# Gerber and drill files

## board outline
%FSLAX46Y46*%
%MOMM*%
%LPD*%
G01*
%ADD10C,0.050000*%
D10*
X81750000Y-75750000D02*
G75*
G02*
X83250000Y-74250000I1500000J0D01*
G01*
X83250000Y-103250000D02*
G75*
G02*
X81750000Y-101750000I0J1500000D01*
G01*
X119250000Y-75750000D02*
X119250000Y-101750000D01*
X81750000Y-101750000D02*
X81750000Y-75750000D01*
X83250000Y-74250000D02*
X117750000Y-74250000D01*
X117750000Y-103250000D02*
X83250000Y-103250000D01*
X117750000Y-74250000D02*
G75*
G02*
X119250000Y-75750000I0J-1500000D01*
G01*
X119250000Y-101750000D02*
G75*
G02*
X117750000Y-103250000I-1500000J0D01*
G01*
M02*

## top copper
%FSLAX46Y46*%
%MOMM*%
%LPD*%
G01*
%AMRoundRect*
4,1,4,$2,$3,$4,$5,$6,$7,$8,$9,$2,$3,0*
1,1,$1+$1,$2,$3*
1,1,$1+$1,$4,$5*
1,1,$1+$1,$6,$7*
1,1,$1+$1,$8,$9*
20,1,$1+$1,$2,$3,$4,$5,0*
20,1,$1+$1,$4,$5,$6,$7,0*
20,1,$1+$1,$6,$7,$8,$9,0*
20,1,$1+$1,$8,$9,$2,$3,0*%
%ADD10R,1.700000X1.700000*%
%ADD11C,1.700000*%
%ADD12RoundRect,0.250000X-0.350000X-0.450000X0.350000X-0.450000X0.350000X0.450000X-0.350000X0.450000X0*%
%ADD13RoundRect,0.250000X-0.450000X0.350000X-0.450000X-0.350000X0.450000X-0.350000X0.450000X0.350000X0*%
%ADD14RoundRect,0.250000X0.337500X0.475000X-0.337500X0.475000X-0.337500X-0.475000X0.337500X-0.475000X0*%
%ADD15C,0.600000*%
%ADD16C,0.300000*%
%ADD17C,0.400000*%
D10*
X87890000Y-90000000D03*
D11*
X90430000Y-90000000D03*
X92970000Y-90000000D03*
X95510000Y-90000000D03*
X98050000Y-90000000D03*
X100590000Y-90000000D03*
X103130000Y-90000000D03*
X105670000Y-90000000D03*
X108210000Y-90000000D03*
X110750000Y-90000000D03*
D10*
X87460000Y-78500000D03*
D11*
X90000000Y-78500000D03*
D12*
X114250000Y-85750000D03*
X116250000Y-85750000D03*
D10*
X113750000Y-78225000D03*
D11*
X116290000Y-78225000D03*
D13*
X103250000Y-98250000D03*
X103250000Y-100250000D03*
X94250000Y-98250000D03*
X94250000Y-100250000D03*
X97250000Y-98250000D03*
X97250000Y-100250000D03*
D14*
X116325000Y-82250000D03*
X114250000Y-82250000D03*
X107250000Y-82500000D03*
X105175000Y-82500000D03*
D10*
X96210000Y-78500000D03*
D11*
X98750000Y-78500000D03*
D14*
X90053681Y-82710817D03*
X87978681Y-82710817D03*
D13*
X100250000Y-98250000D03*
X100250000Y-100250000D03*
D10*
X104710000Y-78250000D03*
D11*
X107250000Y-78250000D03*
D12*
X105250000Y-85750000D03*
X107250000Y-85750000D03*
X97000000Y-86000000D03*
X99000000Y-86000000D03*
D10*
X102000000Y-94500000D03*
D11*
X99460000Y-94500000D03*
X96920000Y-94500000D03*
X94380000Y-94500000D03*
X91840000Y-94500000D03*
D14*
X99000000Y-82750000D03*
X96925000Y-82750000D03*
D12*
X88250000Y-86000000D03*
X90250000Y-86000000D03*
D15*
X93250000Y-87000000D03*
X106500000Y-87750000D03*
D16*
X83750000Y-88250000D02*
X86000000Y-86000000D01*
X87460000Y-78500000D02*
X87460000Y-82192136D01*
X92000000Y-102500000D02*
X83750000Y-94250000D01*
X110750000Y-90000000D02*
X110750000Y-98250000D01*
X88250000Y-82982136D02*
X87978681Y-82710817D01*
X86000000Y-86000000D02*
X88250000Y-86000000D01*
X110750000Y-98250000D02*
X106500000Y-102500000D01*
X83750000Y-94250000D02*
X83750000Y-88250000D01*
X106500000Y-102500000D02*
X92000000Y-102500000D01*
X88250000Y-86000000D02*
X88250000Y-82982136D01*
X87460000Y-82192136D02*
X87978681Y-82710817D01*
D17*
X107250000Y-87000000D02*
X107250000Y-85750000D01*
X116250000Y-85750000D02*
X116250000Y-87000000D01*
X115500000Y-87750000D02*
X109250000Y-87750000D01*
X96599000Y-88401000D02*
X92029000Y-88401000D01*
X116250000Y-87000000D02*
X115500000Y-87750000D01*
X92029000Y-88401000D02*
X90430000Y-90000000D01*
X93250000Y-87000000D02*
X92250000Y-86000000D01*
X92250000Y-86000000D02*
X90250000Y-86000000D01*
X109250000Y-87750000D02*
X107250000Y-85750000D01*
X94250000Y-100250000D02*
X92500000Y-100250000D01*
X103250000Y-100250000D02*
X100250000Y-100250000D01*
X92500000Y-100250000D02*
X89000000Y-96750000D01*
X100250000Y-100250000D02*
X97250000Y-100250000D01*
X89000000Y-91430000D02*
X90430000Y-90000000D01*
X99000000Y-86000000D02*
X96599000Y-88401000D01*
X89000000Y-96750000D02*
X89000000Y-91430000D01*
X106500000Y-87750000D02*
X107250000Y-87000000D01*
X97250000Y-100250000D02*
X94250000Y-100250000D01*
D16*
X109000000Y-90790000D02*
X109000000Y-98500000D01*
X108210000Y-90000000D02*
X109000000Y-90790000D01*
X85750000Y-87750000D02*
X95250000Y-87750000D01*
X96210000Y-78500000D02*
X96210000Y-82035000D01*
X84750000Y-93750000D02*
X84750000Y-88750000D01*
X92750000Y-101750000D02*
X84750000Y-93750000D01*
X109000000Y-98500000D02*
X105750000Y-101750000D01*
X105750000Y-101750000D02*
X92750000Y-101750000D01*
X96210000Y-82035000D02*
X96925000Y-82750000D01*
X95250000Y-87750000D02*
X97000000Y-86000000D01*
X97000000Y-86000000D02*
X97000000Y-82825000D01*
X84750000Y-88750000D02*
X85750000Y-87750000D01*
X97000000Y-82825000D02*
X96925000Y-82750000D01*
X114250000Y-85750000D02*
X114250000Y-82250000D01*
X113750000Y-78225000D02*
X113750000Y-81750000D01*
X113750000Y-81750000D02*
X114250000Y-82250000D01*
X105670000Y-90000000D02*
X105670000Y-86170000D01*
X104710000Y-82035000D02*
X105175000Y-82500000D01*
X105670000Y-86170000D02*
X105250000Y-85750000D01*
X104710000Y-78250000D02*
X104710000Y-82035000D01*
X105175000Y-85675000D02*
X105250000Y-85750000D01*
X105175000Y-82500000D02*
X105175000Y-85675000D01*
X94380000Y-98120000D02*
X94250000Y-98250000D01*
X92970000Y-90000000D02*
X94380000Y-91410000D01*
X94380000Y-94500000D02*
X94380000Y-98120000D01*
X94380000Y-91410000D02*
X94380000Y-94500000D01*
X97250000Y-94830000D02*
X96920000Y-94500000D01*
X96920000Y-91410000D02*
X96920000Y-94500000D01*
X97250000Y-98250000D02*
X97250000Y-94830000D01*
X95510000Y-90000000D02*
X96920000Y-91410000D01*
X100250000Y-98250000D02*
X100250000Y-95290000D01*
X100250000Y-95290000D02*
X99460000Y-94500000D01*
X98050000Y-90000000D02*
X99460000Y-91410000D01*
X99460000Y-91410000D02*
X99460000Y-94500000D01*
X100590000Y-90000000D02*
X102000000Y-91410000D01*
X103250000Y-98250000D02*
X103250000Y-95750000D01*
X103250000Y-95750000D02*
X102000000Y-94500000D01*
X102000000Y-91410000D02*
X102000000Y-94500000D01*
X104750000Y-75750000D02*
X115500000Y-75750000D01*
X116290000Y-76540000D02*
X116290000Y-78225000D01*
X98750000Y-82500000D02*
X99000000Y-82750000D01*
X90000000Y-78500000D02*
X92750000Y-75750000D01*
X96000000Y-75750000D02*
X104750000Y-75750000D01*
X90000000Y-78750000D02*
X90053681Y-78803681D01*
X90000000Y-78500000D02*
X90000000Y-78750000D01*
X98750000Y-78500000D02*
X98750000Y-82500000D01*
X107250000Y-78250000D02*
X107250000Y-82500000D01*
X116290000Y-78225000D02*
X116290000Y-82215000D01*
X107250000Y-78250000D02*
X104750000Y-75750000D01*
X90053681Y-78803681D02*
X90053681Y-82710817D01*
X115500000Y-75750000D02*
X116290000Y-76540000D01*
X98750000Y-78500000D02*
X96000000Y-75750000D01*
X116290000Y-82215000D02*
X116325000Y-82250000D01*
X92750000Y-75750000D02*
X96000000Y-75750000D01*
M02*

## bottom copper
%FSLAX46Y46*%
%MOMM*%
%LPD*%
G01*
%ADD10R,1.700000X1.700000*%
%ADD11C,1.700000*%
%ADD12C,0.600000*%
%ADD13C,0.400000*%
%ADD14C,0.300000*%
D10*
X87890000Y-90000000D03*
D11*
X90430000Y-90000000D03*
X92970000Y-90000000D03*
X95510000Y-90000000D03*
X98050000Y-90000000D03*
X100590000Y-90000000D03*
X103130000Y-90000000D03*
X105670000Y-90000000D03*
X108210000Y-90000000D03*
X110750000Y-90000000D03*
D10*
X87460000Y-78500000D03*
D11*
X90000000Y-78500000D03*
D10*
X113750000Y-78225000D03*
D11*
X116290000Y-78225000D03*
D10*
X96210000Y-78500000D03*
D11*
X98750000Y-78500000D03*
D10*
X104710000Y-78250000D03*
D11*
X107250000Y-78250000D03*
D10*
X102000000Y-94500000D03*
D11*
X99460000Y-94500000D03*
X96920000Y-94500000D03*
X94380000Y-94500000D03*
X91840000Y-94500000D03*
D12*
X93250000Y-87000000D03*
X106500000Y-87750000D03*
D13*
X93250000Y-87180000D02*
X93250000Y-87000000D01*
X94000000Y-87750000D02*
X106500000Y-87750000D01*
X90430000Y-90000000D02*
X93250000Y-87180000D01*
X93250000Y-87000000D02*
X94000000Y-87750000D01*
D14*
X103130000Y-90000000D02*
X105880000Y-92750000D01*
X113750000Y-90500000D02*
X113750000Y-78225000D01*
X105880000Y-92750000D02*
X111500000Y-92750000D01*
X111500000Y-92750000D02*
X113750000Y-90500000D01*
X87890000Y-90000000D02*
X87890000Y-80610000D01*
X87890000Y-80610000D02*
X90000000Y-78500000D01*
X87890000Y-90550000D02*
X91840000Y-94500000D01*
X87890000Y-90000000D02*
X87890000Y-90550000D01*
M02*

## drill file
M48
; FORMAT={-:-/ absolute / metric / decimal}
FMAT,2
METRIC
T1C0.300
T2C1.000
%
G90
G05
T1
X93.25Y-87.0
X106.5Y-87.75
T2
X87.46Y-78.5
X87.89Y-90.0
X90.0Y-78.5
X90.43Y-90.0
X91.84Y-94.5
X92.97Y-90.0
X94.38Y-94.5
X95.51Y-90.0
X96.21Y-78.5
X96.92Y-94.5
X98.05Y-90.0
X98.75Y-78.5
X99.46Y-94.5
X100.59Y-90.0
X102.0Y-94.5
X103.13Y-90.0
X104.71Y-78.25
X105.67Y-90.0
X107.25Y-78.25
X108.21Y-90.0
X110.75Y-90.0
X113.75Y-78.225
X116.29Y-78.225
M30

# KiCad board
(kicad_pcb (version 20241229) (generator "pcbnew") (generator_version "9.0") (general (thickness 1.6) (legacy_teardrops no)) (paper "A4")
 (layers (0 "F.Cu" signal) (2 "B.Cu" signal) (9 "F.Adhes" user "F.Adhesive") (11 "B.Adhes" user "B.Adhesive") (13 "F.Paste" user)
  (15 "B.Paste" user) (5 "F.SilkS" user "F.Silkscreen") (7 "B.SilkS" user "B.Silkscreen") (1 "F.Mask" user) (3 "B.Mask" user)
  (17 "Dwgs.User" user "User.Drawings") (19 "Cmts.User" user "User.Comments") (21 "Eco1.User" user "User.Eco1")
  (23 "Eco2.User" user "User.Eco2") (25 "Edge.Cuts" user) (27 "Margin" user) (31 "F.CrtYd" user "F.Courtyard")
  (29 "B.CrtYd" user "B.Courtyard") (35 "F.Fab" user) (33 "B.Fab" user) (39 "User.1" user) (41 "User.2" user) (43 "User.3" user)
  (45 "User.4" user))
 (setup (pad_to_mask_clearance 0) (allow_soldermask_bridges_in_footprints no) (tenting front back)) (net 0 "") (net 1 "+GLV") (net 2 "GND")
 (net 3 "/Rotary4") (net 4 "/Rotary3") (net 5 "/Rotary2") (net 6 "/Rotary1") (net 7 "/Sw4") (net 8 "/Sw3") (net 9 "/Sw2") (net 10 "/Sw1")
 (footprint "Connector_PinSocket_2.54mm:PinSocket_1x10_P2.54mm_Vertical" (layer "F.Cu") (at 87.89 90 90)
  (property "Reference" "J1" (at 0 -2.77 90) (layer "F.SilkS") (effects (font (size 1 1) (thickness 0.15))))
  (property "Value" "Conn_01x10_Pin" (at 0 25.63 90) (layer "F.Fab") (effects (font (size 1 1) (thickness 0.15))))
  (pad "1" thru_hole rect (at 0 0 90) (size 1.7 1.7) (drill 1) (layers "*.Cu" "*.Mask") (remove_unused_layers no) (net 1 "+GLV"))
  (pad "2" thru_hole circle (at 0 2.54 90) (size 1.7 1.7) (drill 1) (layers "*.Cu" "*.Mask") (remove_unused_layers no) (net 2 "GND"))
  (pad "3" thru_hole circle (at 0 5.08 90) (size 1.7 1.7) (drill 1) (layers "*.Cu" "*.Mask") (remove_unused_layers no) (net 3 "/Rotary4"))
  (pad "4" thru_hole circle (at 0 7.62 90) (size 1.7 1.7) (drill 1) (layers "*.Cu" "*.Mask") (remove_unused_layers no) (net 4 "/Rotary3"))
  (pad "5" thru_hole circle (at 0 10.16 90) (size 1.7 1.7) (drill 1) (layers "*.Cu" "*.Mask") (remove_unused_layers no) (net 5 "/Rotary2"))
  (pad "6" thru_hole circle (at 0 12.7 90) (size 1.7 1.7) (drill 1) (layers "*.Cu" "*.Mask") (remove_unused_layers no) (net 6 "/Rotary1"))
  (pad "7" thru_hole circle (at 0 15.24 90) (size 1.7 1.7) (drill 1) (layers "*.Cu" "*.Mask") (remove_unused_layers no) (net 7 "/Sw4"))
  (pad "8" thru_hole circle (at 0 17.78 90) (size 1.7 1.7) (drill 1) (layers "*.Cu" "*.Mask") (remove_unused_layers no) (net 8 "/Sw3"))
  (pad "9" thru_hole circle (at 0 20.32 90) (size 1.7 1.7) (drill 1) (layers "*.Cu" "*.Mask") (remove_unused_layers no) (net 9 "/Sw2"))
  (pad "10" thru_hole circle (at 0 22.86 90) (size 1.7 1.7) (drill 1) (layers "*.Cu" "*.Mask") (remove_unused_layers no) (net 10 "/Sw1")))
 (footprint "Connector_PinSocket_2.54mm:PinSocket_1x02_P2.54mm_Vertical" (layer "F.Cu") (at 87.46 78.5 90)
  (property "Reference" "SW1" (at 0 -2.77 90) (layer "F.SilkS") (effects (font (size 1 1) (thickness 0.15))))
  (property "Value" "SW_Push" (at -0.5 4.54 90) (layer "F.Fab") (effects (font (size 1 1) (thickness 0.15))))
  (pad "1" thru_hole rect (at 0 0 90) (size 1.7 1.7) (drill 1) (layers "*.Cu" "*.Mask") (remove_unused_layers no) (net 10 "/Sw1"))
  (pad "2" thru_hole circle (at 0 2.54 90) (size 1.7 1.7) (drill 1) (layers "*.Cu" "*.Mask") (remove_unused_layers no) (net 1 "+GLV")))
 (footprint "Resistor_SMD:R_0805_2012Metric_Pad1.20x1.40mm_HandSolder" (layer "F.Cu") (at 115.25 85.75)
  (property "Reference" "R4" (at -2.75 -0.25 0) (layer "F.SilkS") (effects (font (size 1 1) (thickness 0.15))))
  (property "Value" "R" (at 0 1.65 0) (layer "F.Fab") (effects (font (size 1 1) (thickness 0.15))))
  (pad "1" smd roundrect (at -1 0) (size 1.2 1.4) (layers "F.Cu" "F.Mask" "F.Paste") (roundrect_rratio 0.208333) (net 7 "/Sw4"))
  (pad "2" smd roundrect (at 1 0) (size 1.2 1.4) (layers "F.Cu" "F.Mask" "F.Paste") (roundrect_rratio 0.208333) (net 2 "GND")))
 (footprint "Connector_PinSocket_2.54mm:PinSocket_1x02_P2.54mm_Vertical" (layer "F.Cu") (at 113.75 78.225 90)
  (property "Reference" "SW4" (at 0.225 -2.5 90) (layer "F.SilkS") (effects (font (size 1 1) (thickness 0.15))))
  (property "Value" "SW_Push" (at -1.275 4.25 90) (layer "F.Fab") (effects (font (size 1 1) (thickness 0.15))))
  (pad "1" thru_hole rect (at 0 0 90) (size 1.7 1.7) (drill 1) (layers "*.Cu" "*.Mask") (remove_unused_layers no) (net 7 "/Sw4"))
  (pad "2" thru_hole circle (at 0 2.54 90) (size 1.7 1.7) (drill 1) (layers "*.Cu" "*.Mask") (remove_unused_layers no) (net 1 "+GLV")))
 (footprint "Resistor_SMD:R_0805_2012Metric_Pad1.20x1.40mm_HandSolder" (layer "F.Cu") (at 103.25 99.25 -90)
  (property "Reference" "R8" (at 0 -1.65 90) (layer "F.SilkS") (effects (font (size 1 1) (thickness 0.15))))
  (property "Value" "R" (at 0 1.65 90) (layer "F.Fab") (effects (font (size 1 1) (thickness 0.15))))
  (pad "1" smd roundrect (at -1 0 270) (size 1.2 1.4) (layers "F.Cu" "F.Mask" "F.Paste") (roundrect_rratio 0.208333) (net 6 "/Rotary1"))
  (pad "2" smd roundrect (at 1 0 270) (size 1.2 1.4) (layers "F.Cu" "F.Mask" "F.Paste") (roundrect_rratio 0.208333) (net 2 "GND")))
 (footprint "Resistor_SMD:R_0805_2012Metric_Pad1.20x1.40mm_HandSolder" (layer "F.Cu") (at 94.25 99.25 -90)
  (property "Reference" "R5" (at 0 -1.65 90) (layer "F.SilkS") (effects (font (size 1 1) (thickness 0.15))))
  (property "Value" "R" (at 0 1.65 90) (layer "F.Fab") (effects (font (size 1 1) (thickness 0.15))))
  (pad "1" smd roundrect (at -1 0 270) (size 1.2 1.4) (layers "F.Cu" "F.Mask" "F.Paste") (roundrect_rratio 0.208333) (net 3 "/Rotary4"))
  (pad "2" smd roundrect (at 1 0 270) (size 1.2 1.4) (layers "F.Cu" "F.Mask" "F.Paste") (roundrect_rratio 0.208333) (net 2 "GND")))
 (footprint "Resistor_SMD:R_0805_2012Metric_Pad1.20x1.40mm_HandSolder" (layer "F.Cu") (at 97.25 99.25 -90)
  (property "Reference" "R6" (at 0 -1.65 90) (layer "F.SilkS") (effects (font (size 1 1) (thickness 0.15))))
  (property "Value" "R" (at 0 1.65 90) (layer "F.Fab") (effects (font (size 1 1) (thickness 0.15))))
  (pad "1" smd roundrect (at -1 0 270) (size 1.2 1.4) (layers "F.Cu" "F.Mask" "F.Paste") (roundrect_rratio 0.208333) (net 4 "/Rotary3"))
  (pad "2" smd roundrect (at 1 0 270) (size 1.2 1.4) (layers "F.Cu" "F.Mask" "F.Paste") (roundrect_rratio 0.208333) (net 2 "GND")))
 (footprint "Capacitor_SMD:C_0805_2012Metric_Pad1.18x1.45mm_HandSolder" (layer "F.Cu") (at 115.2875 82.25 180)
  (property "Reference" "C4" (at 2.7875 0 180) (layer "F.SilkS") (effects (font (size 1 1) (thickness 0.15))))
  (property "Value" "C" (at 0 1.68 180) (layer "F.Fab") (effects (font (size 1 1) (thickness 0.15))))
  (pad "1" smd roundrect (at -1.0375 0 180) (size 1.175 1.45) (layers "F.Cu" "F.Mask" "F.Paste") (roundrect_rratio 0.212766) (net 1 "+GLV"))
  (pad "2" smd roundrect (at 1.0375 0 180) (size 1.175 1.45) (layers "F.Cu" "F.Mask" "F.Paste") (roundrect_rratio 0.212766) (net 7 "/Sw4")))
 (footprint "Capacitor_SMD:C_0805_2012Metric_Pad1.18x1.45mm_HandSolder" (layer "F.Cu") (at 106.2125 82.5 180)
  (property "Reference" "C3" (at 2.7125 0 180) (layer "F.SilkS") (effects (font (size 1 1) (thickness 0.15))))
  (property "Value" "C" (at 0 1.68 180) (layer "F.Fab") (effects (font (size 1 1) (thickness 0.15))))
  (pad "1" smd roundrect (at -1.0375 0 180) (size 1.175 1.45) (layers "F.Cu" "F.Mask" "F.Paste") (roundrect_rratio 0.212766) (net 1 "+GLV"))
  (pad "2" smd roundrect (at 1.0375 0 180) (size 1.175 1.45) (layers "F.Cu" "F.Mask" "F.Paste") (roundrect_rratio 0.212766) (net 8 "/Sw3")))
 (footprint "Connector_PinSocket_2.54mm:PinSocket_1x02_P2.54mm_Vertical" (layer "F.Cu") (at 96.21 78.5 90)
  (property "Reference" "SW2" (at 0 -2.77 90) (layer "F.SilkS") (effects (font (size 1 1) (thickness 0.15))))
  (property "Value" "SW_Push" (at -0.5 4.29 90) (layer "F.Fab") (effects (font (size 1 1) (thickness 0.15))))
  (pad "1" thru_hole rect (at 0 0 90) (size 1.7 1.7) (drill 1) (layers "*.Cu" "*.Mask") (remove_unused_layers no) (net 9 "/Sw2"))
  (pad "2" thru_hole circle (at 0 2.54 90) (size 1.7 1.7) (drill 1) (layers "*.Cu" "*.Mask") (remove_unused_layers no) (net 1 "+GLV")))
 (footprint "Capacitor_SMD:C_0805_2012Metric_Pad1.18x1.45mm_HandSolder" (layer "F.Cu") (at 89.016181 82.710817 180)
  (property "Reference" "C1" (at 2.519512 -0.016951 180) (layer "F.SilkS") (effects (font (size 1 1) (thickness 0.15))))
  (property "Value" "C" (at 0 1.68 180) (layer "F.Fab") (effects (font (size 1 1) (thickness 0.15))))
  (pad "1" smd roundrect (at -1.0375 0 180) (size 1.175 1.45) (layers "F.Cu" "F.Mask" "F.Paste") (roundrect_rratio 0.212766) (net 1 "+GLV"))
  (pad "2" smd roundrect (at 1.0375 0 180) (size 1.175 1.45) (layers "F.Cu" "F.Mask" "F.Paste") (roundrect_rratio 0.212766) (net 10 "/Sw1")))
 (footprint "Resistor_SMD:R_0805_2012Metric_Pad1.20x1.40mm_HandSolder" (layer "F.Cu") (at 100.25 99.25 -90)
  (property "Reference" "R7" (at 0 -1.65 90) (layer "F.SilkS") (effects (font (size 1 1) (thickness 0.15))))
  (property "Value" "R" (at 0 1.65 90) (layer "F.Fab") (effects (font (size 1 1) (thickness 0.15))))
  (pad "1" smd roundrect (at -1 0 270) (size 1.2 1.4) (layers "F.Cu" "F.Mask" "F.Paste") (roundrect_rratio 0.208333) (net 5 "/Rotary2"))
  (pad "2" smd roundrect (at 1 0 270) (size 1.2 1.4) (layers "F.Cu" "F.Mask" "F.Paste") (roundrect_rratio 0.208333) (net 2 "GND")))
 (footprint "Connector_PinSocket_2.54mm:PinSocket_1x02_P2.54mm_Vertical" (layer "F.Cu") (at 104.71 78.25 90)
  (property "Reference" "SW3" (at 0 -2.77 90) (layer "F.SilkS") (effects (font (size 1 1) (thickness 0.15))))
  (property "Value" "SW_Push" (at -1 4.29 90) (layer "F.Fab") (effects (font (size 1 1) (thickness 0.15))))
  (pad "1" thru_hole rect (at 0 0 90) (size 1.7 1.7) (drill 1) (layers "*.Cu" "*.Mask") (remove_unused_layers no) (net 8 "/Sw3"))
  (pad "2" thru_hole circle (at 0 2.54 90) (size 1.7 1.7) (drill 1) (layers "*.Cu" "*.Mask") (remove_unused_layers no) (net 1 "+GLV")))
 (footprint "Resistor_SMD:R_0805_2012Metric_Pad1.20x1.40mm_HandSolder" (layer "F.Cu") (at 106.25 85.75)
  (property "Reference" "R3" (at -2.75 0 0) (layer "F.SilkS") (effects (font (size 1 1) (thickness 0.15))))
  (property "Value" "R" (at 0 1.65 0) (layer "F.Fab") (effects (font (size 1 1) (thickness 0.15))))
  (pad "1" smd roundrect (at -1 0) (size 1.2 1.4) (layers "F.Cu" "F.Mask" "F.Paste") (roundrect_rratio 0.208333) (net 8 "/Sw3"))
  (pad "2" smd roundrect (at 1 0) (size 1.2 1.4) (layers "F.Cu" "F.Mask" "F.Paste") (roundrect_rratio 0.208333) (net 2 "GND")))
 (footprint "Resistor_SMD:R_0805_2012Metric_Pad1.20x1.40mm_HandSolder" (layer "F.Cu") (at 98 86)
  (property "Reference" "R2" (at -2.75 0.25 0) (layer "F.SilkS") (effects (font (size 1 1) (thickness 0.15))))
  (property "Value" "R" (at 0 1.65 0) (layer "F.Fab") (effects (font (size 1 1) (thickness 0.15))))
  (pad "1" smd roundrect (at -1 0) (size 1.2 1.4) (layers "F.Cu" "F.Mask" "F.Paste") (roundrect_rratio 0.208333) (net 9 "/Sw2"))
  (pad "2" smd roundrect (at 1 0) (size 1.2 1.4) (layers "F.Cu" "F.Mask" "F.Paste") (roundrect_rratio 0.208333) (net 2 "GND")))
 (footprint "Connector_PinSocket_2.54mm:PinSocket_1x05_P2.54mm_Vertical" (layer "F.Cu") (at 102 94.5 -90)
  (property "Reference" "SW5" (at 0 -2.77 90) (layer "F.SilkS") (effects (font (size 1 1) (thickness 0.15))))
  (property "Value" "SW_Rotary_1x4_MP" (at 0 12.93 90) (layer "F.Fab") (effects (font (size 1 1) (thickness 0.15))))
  (pad "1" thru_hole rect (at 0 0 270) (size 1.7 1.7) (drill 1) (layers "*.Cu" "*.Mask") (remove_unused_layers no) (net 6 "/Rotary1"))
  (pad "2" thru_hole circle (at 0 2.54 270) (size 1.7 1.7) (drill 1) (layers "*.Cu" "*.Mask") (remove_unused_layers no) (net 5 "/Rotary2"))
  (pad "3" thru_hole circle (at 0 5.08 270) (size 1.7 1.7) (drill 1) (layers "*.Cu" "*.Mask") (remove_unused_layers no) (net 4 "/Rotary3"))
  (pad "4" thru_hole circle (at 0 7.62 270) (size 1.7 1.7) (drill 1) (layers "*.Cu" "*.Mask") (remove_unused_layers no) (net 3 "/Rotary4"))
  (pad "5" thru_hole circle (at 0 10.16 270) (size 1.7 1.7) (drill 1) (layers "*.Cu" "*.Mask") (remove_unused_layers no) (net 1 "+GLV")))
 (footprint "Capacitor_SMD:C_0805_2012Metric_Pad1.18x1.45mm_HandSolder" (layer "F.Cu") (at 97.9625 82.75 180)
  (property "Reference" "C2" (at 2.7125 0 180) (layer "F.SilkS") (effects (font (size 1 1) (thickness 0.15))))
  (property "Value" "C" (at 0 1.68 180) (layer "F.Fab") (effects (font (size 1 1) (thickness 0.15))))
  (pad "1" smd roundrect (at -1.0375 0 180) (size 1.175 1.45) (layers "F.Cu" "F.Mask" "F.Paste") (roundrect_rratio 0.212766) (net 1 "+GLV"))
  (pad "2" smd roundrect (at 1.0375 0 180) (size 1.175 1.45) (layers "F.Cu" "F.Mask" "F.Paste") (roundrect_rratio 0.212766) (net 9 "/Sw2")))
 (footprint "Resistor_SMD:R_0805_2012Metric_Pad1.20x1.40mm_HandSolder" (layer "F.Cu") (at 89.25 86)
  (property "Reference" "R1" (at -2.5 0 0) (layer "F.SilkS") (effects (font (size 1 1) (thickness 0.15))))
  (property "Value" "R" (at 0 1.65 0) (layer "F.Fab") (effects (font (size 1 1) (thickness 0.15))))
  (pad "1" smd roundrect (at -1 0) (size 1.2 1.4) (layers "F.Cu" "F.Mask" "F.Paste") (roundrect_rratio 0.208333) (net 10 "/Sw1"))
  (pad "2" smd roundrect (at 1 0) (size 1.2 1.4) (layers "F.Cu" "F.Mask" "F.Paste") (roundrect_rratio 0.208333) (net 2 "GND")))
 (gr_arc (start 81.75 75.75) (mid 82.18934 74.68934) (end 83.25 74.25) (stroke (width 0.05) (type default)) (layer "Edge.Cuts"))
 (gr_arc (start 83.25 103.25) (mid 82.18934 102.81066) (end 81.75 101.75) (stroke (width 0.05) (type default)) (layer "Edge.Cuts"))
 (gr_line (start 119.25 75.75) (end 119.25 101.75) (stroke (width 0.05) (type default)) (layer "Edge.Cuts"))
 (gr_line (start 81.75 101.75) (end 81.75 75.75) (stroke (width 0.05) (type default)) (layer "Edge.Cuts"))
 (gr_line (start 83.25 74.25) (end 117.75 74.25) (stroke (width 0.05) (type default)) (layer "Edge.Cuts"))
 (gr_line (start 117.75 103.25) (end 83.25 103.25) (stroke (width 0.05) (type default)) (layer "Edge.Cuts"))
 (gr_arc (start 117.75 74.25) (mid 118.81066 74.68934) (end 119.25 75.75) (stroke (width 0.05) (type default)) (layer "Edge.Cuts"))
 (gr_arc (start 119.25 101.75) (mid 118.81066 102.81066) (end 117.75 103.25) (stroke (width 0.05) (type default)) (layer "Edge.Cuts"))
 (segment (start 83.75 88.25) (end 86 86) (width 0.3) (layer "F.Cu") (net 10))
 (segment (start 87.46 78.5) (end 87.46 82.192136) (width 0.3) (layer "F.Cu") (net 10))
 (segment (start 92 102.5) (end 83.75 94.25) (width 0.3) (layer "F.Cu") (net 10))
 (segment (start 110.75 90) (end 110.75 98.25) (width 0.3) (layer "F.Cu") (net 10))
 (segment (start 88.25 82.982136) (end 87.978681 82.710817) (width 0.3) (layer "F.Cu") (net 10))
 (segment (start 86 86) (end 88.25 86) (width 0.3) (layer "F.Cu") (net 10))
 (segment (start 110.75 98.25) (end 106.5 102.5) (width 0.3) (layer "F.Cu") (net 10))
 (segment (start 83.75 94.25) (end 83.75 88.25) (width 0.3) (layer "F.Cu") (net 10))
 (segment (start 106.5 102.5) (end 92 102.5) (width 0.3) (layer "F.Cu") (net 10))
 (segment (start 88.25 86) (end 88.25 82.982136) (width 0.3) (layer "F.Cu") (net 10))
 (segment (start 87.46 82.192136) (end 87.978681 82.710817) (width 0.3) (layer "F.Cu") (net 10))
 (segment (start 107.25 87) (end 107.25 85.75) (width 0.4) (layer "F.Cu") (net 2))
 (segment (start 116.25 85.75) (end 116.25 87) (width 0.4) (layer "F.Cu") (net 2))
 (segment (start 115.5 87.75) (end 109.25 87.75) (width 0.4) (layer "F.Cu") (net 2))
 (segment (start 96.599 88.401) (end 92.029 88.401) (width 0.4) (layer "F.Cu") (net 2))
 (segment (start 116.25 87) (end 115.5 87.75) (width 0.4) (layer "F.Cu") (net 2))
 (segment (start 92.029 88.401) (end 90.43 90) (width 0.4) (layer "F.Cu") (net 2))
 (segment (start 93.25 87) (end 92.25 86) (width 0.4) (layer "F.Cu") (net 2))
 (segment (start 92.25 86) (end 90.25 86) (width 0.4) (layer "F.Cu") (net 2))
 (segment (start 109.25 87.75) (end 107.25 85.75) (width 0.4) (layer "F.Cu") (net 2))
 (segment (start 94.25 100.25) (end 92.5 100.25) (width 0.4) (layer "F.Cu") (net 2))
 (segment (start 103.25 100.25) (end 100.25 100.25) (width 0.4) (layer "F.Cu") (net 2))
 (segment (start 92.5 100.25) (end 89 96.75) (width 0.4) (layer "F.Cu") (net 2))
 (segment (start 100.25 100.25) (end 97.25 100.25) (width 0.4) (layer "F.Cu") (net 2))
 (segment (start 89 91.43) (end 90.43 90) (width 0.4) (layer "F.Cu") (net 2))
 (segment (start 99 86) (end 96.599 88.401) (width 0.4) (layer "F.Cu") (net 2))
 (segment (start 89 96.75) (end 89 91.43) (width 0.4) (layer "F.Cu") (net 2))
 (segment (start 106.5 87.75) (end 107.25 87) (width 0.4) (layer "F.Cu") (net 2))
 (segment (start 97.25 100.25) (end 94.25 100.25) (width 0.4) (layer "F.Cu") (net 2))
 (via (at 93.25 87) (size 0.6) (drill 0.3) (layers "F.Cu" "B.Cu") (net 2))
 (via (at 106.5 87.75) (size 0.6) (drill 0.3) (layers "F.Cu" "B.Cu") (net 2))
 (segment (start 93.25 87.18) (end 93.25 87) (width 0.4) (layer "B.Cu") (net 2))
 (segment (start 94 87.75) (end 106.5 87.75) (width 0.4) (layer "B.Cu") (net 2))
 (segment (start 90.43 90) (end 93.25 87.18) (width 0.4) (layer "B.Cu") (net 2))
 (segment (start 93.25 87) (end 94 87.75) (width 0.4) (layer "B.Cu") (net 2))
 (segment (start 109 90.79) (end 109 98.5) (width 0.3) (layer "F.Cu") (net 9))
 (segment (start 108.21 90) (end 109 90.79) (width 0.3) (layer "F.Cu") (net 9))
 (segment (start 85.75 87.75) (end 95.25 87.75) (width 0.3) (layer "F.Cu") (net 9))
 (segment (start 96.21 78.5) (end 96.21 82.035) (width 0.3) (layer "F.Cu") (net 9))
 (segment (start 84.75 93.75) (end 84.75 88.75) (width 0.3) (layer "F.Cu") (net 9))
 (segment (start 92.75 101.75) (end 84.75 93.75) (width 0.3) (layer "F.Cu") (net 9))
 (segment (start 109 98.5) (end 105.75 101.75) (width 0.3) (layer "F.Cu") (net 9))
 (segment (start 105.75 101.75) (end 92.75 101.75) (width 0.3) (layer "F.Cu") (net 9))
 (segment (start 96.21 82.035) (end 96.925 82.75) (width 0.3) (layer "F.Cu") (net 9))
 (segment (start 95.25 87.75) (end 97 86) (width 0.3) (layer "F.Cu") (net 9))
 (segment (start 97 86) (end 97 82.825) (width 0.3) (layer "F.Cu") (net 9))
 (segment (start 84.75 88.75) (end 85.75 87.75) (width 0.3) (layer "F.Cu") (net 9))
 (segment (start 97 82.825) (end 96.925 82.75) (width 0.3) (layer "F.Cu") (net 9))
 (segment (start 114.25 85.75) (end 114.25 82.25) (width 0.3) (layer "F.Cu") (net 7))
 (segment (start 113.75 78.225) (end 113.75 81.75) (width 0.3) (layer "F.Cu") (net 7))
 (segment (start 113.75 81.75) (end 114.25 82.25) (width 0.3) (layer "F.Cu") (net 7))
 (segment (start 103.13 90) (end 105.88 92.75) (width 0.3) (layer "B.Cu") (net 7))
 (segment (start 113.75 90.5) (end 113.75 78.225) (width 0.3) (layer "B.Cu") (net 7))
 (segment (start 105.88 92.75) (end 111.5 92.75) (width 0.3) (layer "B.Cu") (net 7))
 (segment (start 111.5 92.75) (end 113.75 90.5) (width 0.3) (layer "B.Cu") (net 7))
 (segment (start 105.67 90) (end 105.67 86.17) (width 0.3) (layer "F.Cu") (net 8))
 (segment (start 104.71 82.035) (end 105.175 82.5) (width 0.3) (layer "F.Cu") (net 8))
 (segment (start 105.67 86.17) (end 105.25 85.75) (width 0.3) (layer "F.Cu") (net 8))
 (segment (start 104.71 78.25) (end 104.71 82.035) (width 0.3) (layer "F.Cu") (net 8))
 (segment (start 105.175 85.675) (end 105.25 85.75) (width 0.3) (layer "F.Cu") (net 8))
 (segment (start 105.175 82.5) (end 105.175 85.675) (width 0.3) (layer "F.Cu") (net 8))
 (segment (start 94.38 98.12) (end 94.25 98.25) (width 0.3) (layer "F.Cu") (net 3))
 (segment (start 92.97 90) (end 94.38 91.41) (width 0.3) (layer "F.Cu") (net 3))
 (segment (start 94.38 94.5) (end 94.38 98.12) (width 0.3) (layer "F.Cu") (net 3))
 (segment (start 94.38 91.41) (end 94.38 94.5) (width 0.3) (layer "F.Cu") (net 3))
 (segment (start 97.25 94.83) (end 96.92 94.5) (width 0.3) (layer "F.Cu") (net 4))
 (segment (start 96.92 91.41) (end 96.92 94.5) (width 0.3) (layer "F.Cu") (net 4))
 (segment (start 97.25 98.25) (end 97.25 94.83) (width 0.3) (layer "F.Cu") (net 4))
 (segment (start 95.51 90) (end 96.92 91.41) (width 0.3) (layer "F.Cu") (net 4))
 (segment (start 100.25 98.25) (end 100.25 95.29) (width 0.3) (layer "F.Cu") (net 5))
 (segment (start 100.25 95.29) (end 99.46 94.5) (width 0.3) (layer "F.Cu") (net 5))
 (segment (start 98.05 90) (end 99.46 91.41) (width 0.3) (layer "F.Cu") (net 5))
 (segment (start 99.46 91.41) (end 99.46 94.5) (width 0.3) (layer "F.Cu") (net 5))
 (segment (start 100.59 90) (end 102 91.41) (width 0.3) (layer "F.Cu") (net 6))
 (segment (start 103.25 98.25) (end 103.25 95.75) (width 0.3) (layer "F.Cu") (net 6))
 (segment (start 103.25 95.75) (end 102 94.5) (width 0.3) (layer "F.Cu") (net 6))
 (segment (start 102 91.41) (end 102 94.5) (width 0.3) (layer "F.Cu") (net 6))
 (segment (start 104.75 75.75) (end 115.5 75.75) (width 0.3) (layer "F.Cu") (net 1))
 (segment (start 116.29 76.54) (end 116.29 78.225) (width 0.3) (layer "F.Cu") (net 1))
 (segment (start 98.75 82.5) (end 99 82.75) (width 0.3) (layer "F.Cu") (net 1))
 (segment (start 90 78.5) (end 92.75 75.75) (width 0.3) (layer "F.Cu") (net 1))
 (segment (start 96 75.75) (end 104.75 75.75) (width 0.3) (layer "F.Cu") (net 1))
 (segment (start 90 78.75) (end 90.053681 78.803681) (width 0.3) (layer "F.Cu") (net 1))
 (segment (start 90 78.5) (end 90 78.75) (width 0.3) (layer "F.Cu") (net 1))
 (segment (start 98.75 78.5) (end 98.75 82.5) (width 0.3) (layer "F.Cu") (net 1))
 (segment (start 107.25 78.25) (end 107.25 82.5) (width 0.3) (layer "F.Cu") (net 1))
 (segment (start 116.29 78.225) (end 116.29 82.215) (width 0.3) (layer "F.Cu") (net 1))
 (segment (start 107.25 78.25) (end 104.75 75.75) (width 0.3) (layer "F.Cu") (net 1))
 (segment (start 90.053681 78.803681) (end 90.053681 82.710817) (width 0.3) (layer "F.Cu") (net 1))
 (segment (start 115.5 75.75) (end 116.29 76.54) (width 0.3) (layer "F.Cu") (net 1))
 (segment (start 98.75 78.5) (end 96 75.75) (width 0.3) (layer "F.Cu") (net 1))
 (segment (start 116.29 82.215) (end 116.325 82.25) (width 0.3) (layer "F.Cu") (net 1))
 (segment (start 92.75 75.75) (end 96 75.75) (width 0.3) (layer "F.Cu") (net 1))
 (segment (start 87.89 90) (end 87.89 80.61) (width 0.3) (layer "B.Cu") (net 1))
 (segment (start 87.89 80.61) (end 90 78.5) (width 0.3) (layer "B.Cu") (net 1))
 (segment (start 87.89 90.55) (end 91.84 94.5) (width 0.3) (layer "B.Cu") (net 1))
 (segment (start 87.89 90) (end 87.89 90.55) (width 0.3) (layer "B.Cu") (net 1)))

